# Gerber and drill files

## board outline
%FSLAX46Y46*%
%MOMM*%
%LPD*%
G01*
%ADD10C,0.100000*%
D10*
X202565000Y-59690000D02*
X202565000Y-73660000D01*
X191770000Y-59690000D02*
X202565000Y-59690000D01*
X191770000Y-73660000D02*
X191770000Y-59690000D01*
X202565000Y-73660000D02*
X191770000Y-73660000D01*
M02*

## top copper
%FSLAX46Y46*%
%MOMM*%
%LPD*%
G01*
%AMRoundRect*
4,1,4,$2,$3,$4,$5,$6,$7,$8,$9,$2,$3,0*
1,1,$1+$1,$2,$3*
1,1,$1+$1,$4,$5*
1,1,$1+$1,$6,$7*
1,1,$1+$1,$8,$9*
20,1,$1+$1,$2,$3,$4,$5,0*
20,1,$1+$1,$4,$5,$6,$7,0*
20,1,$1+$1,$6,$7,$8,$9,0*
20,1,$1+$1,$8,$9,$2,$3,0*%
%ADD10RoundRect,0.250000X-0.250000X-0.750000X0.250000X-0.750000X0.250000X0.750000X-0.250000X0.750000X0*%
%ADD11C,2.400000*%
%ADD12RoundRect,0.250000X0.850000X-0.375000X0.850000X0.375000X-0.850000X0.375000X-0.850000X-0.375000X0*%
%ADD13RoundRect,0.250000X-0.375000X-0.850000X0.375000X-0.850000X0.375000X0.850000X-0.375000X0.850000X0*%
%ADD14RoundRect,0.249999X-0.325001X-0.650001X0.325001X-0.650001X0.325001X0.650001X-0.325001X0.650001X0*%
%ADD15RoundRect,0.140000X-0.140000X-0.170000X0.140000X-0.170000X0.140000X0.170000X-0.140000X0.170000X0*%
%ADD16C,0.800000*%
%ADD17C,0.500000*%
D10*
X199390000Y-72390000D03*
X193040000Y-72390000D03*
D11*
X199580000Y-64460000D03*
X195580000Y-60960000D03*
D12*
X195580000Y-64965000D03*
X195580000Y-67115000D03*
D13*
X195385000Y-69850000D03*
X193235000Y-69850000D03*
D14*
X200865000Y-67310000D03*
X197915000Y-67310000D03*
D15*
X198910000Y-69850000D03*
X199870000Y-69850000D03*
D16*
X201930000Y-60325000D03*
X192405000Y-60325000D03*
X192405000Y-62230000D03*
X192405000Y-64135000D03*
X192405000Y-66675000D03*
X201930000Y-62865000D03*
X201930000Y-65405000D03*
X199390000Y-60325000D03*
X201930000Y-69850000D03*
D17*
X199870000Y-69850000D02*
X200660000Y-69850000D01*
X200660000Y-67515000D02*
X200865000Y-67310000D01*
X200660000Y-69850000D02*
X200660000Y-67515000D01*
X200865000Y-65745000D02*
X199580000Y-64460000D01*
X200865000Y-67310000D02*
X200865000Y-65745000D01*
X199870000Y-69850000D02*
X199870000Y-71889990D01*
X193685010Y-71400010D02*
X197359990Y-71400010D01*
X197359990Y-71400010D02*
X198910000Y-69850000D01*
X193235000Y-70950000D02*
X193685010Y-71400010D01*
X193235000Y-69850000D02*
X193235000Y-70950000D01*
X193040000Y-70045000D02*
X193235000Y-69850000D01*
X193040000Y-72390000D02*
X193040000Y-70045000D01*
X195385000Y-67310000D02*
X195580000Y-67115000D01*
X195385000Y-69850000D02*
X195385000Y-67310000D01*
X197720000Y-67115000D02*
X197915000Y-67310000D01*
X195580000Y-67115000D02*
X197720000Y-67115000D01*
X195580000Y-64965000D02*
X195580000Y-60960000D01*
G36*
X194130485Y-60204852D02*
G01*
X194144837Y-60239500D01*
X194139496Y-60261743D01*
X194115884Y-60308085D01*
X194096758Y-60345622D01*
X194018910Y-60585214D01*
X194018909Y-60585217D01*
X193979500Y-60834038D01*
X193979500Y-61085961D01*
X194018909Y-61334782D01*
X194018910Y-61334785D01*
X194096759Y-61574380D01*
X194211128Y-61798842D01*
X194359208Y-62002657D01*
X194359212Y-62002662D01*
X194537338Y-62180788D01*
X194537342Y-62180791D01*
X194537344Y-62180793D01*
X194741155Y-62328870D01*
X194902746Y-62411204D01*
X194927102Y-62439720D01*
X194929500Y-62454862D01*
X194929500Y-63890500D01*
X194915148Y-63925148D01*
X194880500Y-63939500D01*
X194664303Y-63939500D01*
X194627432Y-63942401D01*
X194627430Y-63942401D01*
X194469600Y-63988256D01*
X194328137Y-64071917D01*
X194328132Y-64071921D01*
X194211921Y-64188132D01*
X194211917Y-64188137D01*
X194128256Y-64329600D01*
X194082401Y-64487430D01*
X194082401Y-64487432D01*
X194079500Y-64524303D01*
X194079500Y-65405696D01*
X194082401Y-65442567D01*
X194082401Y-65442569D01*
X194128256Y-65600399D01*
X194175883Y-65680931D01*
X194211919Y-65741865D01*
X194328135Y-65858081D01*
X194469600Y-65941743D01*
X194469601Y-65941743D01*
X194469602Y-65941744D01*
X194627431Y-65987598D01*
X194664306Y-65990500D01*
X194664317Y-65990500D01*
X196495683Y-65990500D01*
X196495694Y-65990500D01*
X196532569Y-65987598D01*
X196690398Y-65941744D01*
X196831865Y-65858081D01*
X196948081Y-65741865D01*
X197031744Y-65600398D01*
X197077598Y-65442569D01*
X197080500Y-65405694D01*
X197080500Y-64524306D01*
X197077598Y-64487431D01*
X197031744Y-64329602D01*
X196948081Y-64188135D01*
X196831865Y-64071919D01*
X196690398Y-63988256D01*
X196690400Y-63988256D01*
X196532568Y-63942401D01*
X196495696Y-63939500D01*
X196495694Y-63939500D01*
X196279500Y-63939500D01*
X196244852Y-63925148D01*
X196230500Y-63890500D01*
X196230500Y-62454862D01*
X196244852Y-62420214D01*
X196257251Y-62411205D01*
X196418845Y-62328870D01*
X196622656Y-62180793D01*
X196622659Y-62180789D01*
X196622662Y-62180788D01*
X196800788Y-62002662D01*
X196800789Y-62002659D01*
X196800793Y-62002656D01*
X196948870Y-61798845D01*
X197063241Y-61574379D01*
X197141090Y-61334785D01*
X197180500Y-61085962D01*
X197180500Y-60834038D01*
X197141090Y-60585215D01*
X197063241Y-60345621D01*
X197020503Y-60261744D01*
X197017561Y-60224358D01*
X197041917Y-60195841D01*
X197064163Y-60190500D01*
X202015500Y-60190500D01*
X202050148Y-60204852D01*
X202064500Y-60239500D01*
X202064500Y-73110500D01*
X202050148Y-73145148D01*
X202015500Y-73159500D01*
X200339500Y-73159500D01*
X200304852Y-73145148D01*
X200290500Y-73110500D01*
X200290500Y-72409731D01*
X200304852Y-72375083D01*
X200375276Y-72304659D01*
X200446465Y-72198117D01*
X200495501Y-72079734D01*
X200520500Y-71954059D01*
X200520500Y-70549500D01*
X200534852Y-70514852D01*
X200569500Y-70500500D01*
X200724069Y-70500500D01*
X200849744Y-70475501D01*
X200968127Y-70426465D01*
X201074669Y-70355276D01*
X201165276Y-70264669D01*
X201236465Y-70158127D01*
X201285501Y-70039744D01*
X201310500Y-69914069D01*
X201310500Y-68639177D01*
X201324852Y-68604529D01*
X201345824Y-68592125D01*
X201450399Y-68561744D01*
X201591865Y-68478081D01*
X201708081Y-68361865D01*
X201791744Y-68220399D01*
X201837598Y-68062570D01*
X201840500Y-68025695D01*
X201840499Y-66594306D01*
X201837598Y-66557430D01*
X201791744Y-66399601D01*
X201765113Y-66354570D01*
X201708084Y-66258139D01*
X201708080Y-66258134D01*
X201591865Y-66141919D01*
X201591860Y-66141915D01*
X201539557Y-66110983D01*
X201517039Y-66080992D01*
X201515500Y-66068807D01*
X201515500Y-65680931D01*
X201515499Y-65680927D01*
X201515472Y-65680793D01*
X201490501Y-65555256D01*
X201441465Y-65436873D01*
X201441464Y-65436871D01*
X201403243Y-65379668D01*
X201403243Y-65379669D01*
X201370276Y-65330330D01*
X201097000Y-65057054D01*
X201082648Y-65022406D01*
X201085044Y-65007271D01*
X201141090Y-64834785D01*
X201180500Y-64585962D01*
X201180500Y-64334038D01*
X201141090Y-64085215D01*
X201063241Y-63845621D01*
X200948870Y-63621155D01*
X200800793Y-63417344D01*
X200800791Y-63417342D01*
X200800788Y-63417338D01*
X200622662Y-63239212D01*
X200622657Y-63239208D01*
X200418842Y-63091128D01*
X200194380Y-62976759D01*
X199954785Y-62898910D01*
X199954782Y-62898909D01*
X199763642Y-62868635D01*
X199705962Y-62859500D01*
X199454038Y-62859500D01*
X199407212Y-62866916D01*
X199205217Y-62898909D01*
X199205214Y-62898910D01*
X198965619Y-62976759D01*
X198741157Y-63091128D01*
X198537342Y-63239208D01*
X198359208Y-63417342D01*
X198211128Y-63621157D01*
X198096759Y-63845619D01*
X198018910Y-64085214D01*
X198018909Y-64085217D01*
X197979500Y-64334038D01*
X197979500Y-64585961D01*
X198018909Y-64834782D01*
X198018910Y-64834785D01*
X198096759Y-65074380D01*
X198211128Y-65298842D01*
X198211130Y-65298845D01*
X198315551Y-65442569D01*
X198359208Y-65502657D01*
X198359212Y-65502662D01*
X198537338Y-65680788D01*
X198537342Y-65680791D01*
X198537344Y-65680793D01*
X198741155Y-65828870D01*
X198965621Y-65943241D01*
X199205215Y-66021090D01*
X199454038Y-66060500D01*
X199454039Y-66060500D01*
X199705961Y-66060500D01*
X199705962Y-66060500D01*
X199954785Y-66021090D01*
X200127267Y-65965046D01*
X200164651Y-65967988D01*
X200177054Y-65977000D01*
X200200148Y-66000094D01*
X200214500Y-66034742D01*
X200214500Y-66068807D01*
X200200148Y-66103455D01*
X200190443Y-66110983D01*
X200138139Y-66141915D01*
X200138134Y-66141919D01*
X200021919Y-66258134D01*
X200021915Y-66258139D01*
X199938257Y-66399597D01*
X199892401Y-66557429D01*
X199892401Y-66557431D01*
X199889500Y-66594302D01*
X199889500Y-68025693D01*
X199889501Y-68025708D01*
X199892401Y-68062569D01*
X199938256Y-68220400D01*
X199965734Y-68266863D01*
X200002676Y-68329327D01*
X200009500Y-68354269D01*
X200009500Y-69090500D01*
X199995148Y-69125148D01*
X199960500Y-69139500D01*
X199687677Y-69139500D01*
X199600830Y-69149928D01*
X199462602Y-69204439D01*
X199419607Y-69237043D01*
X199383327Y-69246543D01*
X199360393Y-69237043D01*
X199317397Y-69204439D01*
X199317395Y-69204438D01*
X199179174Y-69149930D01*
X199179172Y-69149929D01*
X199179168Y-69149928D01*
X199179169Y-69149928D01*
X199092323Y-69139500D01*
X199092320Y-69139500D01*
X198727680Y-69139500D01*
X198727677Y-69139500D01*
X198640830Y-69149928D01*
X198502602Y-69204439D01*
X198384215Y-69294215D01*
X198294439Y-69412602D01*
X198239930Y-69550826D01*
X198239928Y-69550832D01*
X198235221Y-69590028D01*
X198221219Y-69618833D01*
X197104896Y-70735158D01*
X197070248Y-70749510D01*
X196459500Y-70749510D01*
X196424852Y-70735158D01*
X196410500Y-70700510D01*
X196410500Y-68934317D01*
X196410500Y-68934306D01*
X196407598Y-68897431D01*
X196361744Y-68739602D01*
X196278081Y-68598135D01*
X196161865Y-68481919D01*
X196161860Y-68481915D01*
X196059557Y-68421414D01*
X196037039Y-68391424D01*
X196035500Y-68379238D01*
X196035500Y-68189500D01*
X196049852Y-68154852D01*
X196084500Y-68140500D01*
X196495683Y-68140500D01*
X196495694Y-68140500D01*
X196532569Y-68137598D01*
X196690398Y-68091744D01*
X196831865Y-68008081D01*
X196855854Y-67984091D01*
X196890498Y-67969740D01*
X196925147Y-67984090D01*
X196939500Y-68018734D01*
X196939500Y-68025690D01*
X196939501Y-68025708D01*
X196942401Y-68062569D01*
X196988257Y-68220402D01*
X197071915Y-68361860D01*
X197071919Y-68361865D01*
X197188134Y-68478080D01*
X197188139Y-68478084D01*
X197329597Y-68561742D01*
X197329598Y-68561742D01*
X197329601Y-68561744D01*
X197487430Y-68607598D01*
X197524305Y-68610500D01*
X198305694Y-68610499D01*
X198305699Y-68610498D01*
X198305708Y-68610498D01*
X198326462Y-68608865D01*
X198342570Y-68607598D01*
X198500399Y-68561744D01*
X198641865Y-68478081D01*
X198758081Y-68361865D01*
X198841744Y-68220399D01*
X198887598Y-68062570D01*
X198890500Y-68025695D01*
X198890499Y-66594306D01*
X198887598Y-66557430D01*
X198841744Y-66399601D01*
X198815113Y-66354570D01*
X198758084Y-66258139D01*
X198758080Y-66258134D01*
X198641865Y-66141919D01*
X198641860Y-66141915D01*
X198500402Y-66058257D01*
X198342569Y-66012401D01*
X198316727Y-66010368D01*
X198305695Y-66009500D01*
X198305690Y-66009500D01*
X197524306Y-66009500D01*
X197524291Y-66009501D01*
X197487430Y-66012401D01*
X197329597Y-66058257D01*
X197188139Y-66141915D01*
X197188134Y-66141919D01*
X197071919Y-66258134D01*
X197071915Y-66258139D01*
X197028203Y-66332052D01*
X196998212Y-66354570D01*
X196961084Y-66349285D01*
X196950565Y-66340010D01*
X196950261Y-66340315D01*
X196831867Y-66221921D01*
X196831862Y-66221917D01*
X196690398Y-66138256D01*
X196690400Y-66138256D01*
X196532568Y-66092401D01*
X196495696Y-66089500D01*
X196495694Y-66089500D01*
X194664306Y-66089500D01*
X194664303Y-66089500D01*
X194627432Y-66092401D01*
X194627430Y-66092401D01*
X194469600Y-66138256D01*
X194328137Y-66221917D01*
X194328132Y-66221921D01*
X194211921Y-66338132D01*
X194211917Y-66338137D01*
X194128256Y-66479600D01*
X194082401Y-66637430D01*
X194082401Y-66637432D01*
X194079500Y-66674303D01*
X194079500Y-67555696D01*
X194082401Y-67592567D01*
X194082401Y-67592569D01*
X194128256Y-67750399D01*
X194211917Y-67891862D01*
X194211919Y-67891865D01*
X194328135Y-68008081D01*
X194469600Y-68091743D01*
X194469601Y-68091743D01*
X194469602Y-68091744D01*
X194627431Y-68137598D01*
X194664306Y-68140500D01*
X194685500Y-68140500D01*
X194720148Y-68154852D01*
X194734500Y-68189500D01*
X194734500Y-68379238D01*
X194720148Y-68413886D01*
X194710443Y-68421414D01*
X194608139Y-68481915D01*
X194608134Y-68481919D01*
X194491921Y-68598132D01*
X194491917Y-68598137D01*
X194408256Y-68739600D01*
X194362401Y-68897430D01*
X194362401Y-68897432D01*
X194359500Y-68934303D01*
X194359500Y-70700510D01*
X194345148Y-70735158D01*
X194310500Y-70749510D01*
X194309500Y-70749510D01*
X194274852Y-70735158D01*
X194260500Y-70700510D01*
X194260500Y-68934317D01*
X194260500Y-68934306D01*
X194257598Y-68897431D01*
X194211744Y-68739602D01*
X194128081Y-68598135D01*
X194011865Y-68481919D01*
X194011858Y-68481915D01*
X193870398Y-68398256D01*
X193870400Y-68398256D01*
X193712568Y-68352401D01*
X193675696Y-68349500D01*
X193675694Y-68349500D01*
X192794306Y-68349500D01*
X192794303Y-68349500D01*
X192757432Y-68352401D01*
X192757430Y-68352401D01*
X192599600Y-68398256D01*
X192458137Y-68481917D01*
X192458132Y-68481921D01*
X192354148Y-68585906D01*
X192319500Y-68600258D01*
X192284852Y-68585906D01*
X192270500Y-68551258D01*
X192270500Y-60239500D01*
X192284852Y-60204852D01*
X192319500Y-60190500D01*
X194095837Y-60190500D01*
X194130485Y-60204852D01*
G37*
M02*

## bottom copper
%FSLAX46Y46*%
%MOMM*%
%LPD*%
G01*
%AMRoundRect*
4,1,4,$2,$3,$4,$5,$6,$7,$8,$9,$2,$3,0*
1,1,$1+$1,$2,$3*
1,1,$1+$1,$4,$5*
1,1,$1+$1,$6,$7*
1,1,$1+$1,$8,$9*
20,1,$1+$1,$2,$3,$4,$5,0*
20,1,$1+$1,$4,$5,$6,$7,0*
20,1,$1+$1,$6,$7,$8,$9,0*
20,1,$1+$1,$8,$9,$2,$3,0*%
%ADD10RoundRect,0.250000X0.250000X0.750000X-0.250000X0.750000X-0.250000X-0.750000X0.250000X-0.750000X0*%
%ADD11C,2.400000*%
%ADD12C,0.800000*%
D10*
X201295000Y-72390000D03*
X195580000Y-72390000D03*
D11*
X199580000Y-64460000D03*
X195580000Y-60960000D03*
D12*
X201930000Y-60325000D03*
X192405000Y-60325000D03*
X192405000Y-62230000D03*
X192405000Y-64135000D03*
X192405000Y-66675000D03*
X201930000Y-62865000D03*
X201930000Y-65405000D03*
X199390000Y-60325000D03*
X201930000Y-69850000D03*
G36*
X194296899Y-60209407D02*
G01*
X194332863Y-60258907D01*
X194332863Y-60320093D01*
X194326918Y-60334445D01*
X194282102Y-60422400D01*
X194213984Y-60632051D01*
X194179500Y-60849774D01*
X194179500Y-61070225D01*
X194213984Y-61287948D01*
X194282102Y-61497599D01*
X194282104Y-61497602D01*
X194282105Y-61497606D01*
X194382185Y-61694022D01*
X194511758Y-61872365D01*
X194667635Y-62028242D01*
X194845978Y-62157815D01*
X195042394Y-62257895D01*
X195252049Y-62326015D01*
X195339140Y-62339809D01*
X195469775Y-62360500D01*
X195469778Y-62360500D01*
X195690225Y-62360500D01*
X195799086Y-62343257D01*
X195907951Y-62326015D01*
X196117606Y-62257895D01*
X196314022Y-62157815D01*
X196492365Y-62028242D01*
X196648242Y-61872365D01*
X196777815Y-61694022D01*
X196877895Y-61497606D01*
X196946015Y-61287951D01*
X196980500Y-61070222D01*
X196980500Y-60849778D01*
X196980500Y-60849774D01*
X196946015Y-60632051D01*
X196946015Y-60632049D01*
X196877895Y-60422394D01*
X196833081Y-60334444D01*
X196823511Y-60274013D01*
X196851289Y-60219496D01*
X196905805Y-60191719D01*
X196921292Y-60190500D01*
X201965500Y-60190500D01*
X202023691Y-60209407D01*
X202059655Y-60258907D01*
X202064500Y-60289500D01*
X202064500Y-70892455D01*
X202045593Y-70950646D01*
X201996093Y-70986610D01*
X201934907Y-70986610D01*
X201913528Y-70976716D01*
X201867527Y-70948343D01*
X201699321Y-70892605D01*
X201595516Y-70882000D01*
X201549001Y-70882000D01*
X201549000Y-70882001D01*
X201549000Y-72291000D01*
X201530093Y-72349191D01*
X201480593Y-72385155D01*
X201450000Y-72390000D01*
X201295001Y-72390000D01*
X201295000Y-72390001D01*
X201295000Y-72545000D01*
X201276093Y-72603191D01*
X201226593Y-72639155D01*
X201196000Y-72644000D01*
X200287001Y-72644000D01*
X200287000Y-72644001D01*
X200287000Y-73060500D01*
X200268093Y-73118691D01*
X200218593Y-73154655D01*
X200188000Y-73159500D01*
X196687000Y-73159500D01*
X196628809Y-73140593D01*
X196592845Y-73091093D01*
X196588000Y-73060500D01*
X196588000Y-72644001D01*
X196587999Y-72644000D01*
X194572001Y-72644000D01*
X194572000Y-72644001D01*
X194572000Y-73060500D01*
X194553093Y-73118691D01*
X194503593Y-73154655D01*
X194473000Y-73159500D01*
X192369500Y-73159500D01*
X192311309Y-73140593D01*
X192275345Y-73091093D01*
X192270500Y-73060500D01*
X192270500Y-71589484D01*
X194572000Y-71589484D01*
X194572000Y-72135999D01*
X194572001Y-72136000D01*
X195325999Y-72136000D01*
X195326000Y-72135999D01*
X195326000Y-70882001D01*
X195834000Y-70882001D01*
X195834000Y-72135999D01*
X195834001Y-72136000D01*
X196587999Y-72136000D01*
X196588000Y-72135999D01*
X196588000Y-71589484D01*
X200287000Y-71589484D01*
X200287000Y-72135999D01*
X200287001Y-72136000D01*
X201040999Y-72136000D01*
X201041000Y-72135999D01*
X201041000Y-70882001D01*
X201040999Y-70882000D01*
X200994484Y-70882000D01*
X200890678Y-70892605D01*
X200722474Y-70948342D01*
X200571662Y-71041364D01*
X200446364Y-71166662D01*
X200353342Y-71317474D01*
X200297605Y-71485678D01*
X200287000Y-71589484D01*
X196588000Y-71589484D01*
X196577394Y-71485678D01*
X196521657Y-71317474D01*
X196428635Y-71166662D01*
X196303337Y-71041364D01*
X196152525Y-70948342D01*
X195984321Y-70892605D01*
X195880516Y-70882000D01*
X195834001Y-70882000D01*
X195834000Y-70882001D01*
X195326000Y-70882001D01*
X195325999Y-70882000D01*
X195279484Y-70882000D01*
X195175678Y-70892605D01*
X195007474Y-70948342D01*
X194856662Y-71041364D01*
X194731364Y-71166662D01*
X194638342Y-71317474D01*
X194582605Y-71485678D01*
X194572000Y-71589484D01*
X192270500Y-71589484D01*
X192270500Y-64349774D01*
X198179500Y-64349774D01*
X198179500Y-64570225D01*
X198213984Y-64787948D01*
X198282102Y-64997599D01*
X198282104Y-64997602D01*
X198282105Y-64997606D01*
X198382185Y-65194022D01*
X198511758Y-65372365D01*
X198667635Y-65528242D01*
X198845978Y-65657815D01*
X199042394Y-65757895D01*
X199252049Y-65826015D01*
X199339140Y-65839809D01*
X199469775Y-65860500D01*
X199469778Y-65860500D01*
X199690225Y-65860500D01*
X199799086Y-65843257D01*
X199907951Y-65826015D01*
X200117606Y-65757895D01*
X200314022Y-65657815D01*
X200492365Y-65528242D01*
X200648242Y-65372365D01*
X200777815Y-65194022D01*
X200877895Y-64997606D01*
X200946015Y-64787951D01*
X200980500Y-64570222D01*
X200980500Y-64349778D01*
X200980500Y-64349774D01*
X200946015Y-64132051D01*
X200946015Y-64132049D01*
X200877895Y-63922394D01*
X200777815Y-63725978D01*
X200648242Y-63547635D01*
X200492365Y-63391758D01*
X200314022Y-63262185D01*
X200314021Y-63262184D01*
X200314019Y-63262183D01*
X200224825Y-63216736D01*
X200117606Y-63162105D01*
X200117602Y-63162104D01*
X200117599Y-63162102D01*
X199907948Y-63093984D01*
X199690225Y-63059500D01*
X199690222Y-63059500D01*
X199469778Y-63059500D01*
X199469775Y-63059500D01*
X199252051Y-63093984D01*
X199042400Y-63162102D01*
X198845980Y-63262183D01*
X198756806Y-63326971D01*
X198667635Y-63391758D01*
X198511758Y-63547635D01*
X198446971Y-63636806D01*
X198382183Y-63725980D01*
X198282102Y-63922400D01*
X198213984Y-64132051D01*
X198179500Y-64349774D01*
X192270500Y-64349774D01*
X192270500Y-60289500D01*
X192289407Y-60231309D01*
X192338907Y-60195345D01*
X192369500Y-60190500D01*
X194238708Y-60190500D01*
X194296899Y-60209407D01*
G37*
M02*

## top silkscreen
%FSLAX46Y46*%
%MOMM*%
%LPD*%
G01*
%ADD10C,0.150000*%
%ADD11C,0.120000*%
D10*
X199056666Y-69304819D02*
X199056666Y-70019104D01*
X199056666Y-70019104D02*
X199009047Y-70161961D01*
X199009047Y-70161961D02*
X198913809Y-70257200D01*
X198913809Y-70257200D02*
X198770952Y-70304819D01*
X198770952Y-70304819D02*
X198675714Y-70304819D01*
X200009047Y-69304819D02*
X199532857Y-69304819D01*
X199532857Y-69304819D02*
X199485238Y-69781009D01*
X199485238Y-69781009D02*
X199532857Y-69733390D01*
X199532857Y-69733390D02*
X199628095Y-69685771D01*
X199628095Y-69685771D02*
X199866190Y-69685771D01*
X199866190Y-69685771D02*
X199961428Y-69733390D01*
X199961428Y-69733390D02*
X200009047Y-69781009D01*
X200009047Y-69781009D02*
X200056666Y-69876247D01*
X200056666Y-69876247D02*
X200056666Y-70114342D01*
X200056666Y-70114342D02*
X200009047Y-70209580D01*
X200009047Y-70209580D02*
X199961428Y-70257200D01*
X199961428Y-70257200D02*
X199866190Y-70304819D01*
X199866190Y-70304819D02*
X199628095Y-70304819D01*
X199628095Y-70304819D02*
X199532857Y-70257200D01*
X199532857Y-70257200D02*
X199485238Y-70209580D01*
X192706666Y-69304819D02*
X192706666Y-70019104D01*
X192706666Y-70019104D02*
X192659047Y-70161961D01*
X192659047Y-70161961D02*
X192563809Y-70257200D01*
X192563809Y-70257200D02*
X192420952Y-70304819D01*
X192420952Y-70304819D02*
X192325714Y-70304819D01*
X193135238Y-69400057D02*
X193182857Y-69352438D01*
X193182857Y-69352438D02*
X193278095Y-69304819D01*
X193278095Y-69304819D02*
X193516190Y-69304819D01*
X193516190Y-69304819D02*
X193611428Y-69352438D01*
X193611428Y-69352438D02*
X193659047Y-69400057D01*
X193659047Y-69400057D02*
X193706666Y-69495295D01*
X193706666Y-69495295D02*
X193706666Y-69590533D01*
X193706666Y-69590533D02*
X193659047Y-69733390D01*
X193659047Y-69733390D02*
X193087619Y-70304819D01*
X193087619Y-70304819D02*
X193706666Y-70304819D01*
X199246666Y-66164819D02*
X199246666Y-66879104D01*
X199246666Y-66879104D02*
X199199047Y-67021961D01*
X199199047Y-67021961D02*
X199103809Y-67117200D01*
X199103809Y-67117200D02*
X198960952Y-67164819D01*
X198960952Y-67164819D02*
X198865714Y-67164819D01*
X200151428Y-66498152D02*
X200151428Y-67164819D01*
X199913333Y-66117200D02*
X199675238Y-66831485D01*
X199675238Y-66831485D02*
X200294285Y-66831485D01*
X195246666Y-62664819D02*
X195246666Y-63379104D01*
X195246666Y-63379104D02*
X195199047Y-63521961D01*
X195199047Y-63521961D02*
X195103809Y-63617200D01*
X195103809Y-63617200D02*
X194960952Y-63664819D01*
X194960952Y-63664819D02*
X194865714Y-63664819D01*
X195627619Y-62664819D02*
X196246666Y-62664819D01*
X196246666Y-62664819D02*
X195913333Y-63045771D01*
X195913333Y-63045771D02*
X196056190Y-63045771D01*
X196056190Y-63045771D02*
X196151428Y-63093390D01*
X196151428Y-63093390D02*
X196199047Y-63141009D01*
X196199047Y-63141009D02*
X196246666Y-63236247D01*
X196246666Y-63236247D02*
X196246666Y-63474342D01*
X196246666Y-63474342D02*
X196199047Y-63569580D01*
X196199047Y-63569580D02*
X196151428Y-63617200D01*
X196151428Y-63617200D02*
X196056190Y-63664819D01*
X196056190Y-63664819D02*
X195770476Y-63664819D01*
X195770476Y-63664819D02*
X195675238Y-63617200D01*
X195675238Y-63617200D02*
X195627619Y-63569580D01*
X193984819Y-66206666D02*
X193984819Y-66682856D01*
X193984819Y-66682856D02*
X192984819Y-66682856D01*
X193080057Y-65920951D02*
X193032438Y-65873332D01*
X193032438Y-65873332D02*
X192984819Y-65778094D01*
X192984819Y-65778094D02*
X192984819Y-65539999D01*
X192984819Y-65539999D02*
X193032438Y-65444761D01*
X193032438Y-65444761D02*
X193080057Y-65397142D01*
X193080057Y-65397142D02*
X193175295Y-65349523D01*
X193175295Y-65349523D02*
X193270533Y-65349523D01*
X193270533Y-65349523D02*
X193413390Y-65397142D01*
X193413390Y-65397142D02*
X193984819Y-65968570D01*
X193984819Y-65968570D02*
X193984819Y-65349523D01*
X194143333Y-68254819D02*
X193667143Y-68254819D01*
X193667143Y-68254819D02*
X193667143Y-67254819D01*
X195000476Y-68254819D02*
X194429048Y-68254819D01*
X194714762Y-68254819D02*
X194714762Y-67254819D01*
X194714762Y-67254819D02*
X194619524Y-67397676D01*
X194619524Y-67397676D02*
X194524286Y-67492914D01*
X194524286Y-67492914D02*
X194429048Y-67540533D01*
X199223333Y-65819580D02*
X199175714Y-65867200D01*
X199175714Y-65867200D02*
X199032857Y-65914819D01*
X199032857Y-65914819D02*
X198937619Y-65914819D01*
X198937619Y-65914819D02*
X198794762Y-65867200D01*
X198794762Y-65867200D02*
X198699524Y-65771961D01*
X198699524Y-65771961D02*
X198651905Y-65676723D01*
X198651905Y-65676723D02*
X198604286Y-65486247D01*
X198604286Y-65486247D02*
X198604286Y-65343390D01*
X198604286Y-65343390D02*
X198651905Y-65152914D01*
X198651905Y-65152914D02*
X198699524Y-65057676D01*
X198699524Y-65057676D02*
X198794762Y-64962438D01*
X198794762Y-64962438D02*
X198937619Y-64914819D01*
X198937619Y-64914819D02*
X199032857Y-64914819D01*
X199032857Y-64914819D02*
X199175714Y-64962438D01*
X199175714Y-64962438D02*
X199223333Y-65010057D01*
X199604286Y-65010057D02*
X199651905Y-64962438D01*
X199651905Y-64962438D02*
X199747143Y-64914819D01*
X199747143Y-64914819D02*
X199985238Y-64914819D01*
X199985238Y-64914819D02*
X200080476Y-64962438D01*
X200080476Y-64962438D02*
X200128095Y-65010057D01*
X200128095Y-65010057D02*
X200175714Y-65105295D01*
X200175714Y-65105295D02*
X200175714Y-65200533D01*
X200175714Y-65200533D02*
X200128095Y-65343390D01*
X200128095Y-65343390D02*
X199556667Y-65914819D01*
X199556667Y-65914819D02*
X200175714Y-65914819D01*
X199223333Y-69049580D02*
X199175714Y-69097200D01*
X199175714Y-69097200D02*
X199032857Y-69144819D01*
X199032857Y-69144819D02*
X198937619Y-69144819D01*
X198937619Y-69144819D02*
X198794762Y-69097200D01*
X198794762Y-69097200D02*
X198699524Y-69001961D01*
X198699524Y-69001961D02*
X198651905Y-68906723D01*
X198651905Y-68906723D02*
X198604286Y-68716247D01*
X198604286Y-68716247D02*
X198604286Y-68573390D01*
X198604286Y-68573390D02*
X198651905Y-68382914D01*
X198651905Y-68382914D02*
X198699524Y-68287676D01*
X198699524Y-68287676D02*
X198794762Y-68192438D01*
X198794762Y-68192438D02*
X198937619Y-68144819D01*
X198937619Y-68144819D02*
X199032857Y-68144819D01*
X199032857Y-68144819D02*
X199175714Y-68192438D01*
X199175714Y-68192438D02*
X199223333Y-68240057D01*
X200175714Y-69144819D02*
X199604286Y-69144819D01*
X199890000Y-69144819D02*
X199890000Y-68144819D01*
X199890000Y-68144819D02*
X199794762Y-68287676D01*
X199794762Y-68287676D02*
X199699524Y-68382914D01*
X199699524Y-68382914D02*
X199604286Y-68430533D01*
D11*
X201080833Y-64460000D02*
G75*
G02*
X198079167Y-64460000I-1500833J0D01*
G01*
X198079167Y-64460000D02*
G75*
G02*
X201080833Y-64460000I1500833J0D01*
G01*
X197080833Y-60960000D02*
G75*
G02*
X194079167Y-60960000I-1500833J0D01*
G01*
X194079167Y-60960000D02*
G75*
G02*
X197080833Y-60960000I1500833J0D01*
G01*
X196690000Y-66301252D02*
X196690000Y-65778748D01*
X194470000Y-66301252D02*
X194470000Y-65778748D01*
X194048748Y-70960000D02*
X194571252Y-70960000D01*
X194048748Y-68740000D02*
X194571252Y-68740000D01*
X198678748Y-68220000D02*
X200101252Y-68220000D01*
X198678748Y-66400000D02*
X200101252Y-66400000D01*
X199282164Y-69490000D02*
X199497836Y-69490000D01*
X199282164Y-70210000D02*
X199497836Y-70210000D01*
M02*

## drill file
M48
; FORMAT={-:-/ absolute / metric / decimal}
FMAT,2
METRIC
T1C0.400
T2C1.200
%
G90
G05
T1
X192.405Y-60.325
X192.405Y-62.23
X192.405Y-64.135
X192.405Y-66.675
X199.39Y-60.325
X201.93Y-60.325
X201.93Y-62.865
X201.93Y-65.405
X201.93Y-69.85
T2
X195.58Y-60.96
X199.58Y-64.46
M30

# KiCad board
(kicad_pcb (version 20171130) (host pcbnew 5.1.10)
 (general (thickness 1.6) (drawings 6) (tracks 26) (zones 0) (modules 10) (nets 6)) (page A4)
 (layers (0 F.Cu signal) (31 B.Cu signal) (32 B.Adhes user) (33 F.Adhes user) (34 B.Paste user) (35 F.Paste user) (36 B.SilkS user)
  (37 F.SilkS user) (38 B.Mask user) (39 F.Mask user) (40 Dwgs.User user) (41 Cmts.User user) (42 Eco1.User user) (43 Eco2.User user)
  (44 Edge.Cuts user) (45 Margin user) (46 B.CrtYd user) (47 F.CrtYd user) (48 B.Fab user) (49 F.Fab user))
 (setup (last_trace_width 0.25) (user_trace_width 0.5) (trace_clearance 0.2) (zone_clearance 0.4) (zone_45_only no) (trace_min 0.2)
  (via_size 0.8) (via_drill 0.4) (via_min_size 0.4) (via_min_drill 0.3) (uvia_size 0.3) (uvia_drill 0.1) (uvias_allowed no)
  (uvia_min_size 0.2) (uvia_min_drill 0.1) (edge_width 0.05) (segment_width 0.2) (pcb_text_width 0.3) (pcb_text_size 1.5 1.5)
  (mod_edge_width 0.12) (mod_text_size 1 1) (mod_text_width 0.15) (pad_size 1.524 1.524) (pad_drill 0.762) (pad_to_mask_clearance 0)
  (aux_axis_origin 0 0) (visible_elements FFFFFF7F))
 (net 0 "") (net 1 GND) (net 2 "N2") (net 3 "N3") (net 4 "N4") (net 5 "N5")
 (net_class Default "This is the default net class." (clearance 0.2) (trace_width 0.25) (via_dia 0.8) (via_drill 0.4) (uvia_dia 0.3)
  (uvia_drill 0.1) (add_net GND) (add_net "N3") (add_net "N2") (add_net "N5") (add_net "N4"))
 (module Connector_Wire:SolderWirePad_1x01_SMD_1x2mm (layer B.Cu) (at 201.295 72.39 180)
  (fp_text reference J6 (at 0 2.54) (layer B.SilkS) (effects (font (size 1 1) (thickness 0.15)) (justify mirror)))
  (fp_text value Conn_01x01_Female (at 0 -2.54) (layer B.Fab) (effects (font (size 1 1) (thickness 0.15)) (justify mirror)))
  (pad 1 smd roundrect (at 0 0 180) (size 1 2) (layers B.Cu B.Paste B.Mask) (roundrect_rratio 0.25) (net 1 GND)))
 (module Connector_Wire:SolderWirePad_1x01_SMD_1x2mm (layer F.Cu) (at 199.39 72.39)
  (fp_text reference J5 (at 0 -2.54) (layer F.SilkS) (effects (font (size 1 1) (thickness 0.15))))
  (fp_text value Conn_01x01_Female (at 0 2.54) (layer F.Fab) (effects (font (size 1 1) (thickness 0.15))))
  (pad 1 smd roundrect (at 0 0) (size 1 2) (layers F.Cu F.Paste F.Mask) (roundrect_rratio 0.25) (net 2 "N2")))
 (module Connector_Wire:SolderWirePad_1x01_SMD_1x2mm (layer F.Cu) (at 193.04 72.39)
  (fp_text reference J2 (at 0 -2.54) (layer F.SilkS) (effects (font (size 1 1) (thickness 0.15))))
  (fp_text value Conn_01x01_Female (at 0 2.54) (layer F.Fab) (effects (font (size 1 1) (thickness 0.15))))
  (pad 1 smd roundrect (at 0 0) (size 1 2) (layers F.Cu F.Paste F.Mask) (roundrect_rratio 0.25) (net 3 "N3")))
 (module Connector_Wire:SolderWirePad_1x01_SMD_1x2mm (layer B.Cu) (at 195.58 72.39 180)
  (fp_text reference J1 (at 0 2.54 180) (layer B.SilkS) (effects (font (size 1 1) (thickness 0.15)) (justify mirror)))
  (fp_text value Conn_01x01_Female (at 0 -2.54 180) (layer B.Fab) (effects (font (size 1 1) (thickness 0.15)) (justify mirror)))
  (pad 1 smd roundrect (at 0 0 180) (size 1 2) (layers B.Cu B.Paste B.Mask) (roundrect_rratio 0.25) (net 1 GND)))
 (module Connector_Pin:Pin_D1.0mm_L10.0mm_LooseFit (layer F.Cu) (at 199.58 64.46)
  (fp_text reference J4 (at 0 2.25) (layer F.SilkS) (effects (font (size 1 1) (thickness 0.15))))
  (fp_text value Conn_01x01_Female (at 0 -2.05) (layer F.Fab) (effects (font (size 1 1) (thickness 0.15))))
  (fp_circle (center 0 0) (end 1.5 0.05) (layer F.SilkS) (width 0.12))
  (pad 1 thru_hole circle (at 0 0) (size 2.4 2.4) (drill 1.2) (layers *.Cu *.Mask) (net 2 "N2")))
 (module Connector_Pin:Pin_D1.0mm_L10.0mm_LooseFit (layer F.Cu) (at 195.58 60.96)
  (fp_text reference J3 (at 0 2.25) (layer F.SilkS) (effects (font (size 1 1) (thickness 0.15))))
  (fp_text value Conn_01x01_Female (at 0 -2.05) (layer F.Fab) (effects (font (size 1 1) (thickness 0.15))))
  (fp_circle (center 0 0) (end 1.5 0.05) (layer F.SilkS) (width 0.12))
  (pad 1 thru_hole circle (at 0 0) (size 2.4 2.4) (drill 1.2) (layers *.Cu *.Mask) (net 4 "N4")))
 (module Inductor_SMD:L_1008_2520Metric (layer F.Cu) (at 195.58 66.04 90)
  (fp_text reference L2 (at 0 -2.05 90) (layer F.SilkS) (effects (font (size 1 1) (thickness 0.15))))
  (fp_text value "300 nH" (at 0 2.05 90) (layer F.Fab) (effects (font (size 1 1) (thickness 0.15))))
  (fp_line (start -0.261252 1.11) (end 0.261252 1.11) (layer F.SilkS) (width 0.12))
  (fp_line (start -0.261252 -1.11) (end 0.261252 -1.11) (layer F.SilkS) (width 0.12))
  (pad 2 smd roundrect (at 1.075 0 90) (size 1.25 2.2) (layers F.Cu F.Paste F.Mask) (roundrect_rratio 0.2) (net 4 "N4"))
  (pad 1 smd roundrect (at -1.075 0 90) (size 1.25 2.2) (layers F.Cu F.Paste F.Mask) (roundrect_rratio 0.2) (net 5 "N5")))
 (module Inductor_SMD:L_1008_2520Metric (layer F.Cu) (at 194.31 69.85)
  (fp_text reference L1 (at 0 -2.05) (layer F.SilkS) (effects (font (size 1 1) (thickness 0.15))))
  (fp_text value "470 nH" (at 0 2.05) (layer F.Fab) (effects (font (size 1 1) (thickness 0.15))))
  (fp_line (start -0.261252 1.11) (end 0.261252 1.11) (layer F.SilkS) (width 0.12))
  (fp_line (start -0.261252 -1.11) (end 0.261252 -1.11) (layer F.SilkS) (width 0.12))
  (pad 2 smd roundrect (at 1.075 0) (size 1.25 2.2) (layers F.Cu F.Paste F.Mask) (roundrect_rratio 0.2) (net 5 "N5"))
  (pad 1 smd roundrect (at -1.075 0) (size 1.25 2.2) (layers F.Cu F.Paste F.Mask) (roundrect_rratio 0.2) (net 3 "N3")))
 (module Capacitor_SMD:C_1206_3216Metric (layer F.Cu) (at 199.39 67.31)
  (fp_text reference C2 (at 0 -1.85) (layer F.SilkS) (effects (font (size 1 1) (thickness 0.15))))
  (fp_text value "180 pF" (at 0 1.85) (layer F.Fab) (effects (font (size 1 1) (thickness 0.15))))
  (fp_line (start -0.711252 0.91) (end 0.711252 0.91) (layer F.SilkS) (width 0.12))
  (fp_line (start -0.711252 -0.91) (end 0.711252 -0.91) (layer F.SilkS) (width 0.12))
  (pad 2 smd roundrect (at 1.475 0) (size 1.15 1.8) (layers F.Cu F.Paste F.Mask) (roundrect_rratio 0.2173904347826087) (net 2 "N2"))
  (pad 1 smd roundrect (at -1.475 0) (size 1.15 1.8) (layers F.Cu F.Paste F.Mask) (roundrect_rratio 0.2173904347826087) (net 5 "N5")))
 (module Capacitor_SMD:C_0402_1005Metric (layer F.Cu) (at 199.39 69.85)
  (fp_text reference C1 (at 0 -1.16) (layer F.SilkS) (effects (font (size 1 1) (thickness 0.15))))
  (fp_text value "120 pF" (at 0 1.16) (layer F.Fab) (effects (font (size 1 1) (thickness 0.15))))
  (fp_line (start -0.107836 -0.36) (end 0.107836 -0.36) (layer F.SilkS) (width 0.12))
  (fp_line (start -0.107836 0.36) (end 0.107836 0.36) (layer F.SilkS) (width 0.12))
  (pad 1 smd roundrect (at -0.48 0) (size 0.56 0.62) (layers F.Cu F.Paste F.Mask) (roundrect_rratio 0.25) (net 3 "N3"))
  (pad 2 smd roundrect (at 0.48 0) (size 0.56 0.62) (layers F.Cu F.Paste F.Mask) (roundrect_rratio 0.25) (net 2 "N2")))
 (gr_line (start 202.565 59.69) (end 202.565 73.66) (layer Edge.Cuts) (width 0.1))
 (gr_line (start 191.77 59.69) (end 202.565 59.69) (layer Edge.Cuts) (width 0.1))
 (gr_line (start 191.77 73.66) (end 191.77 59.69) (layer Edge.Cuts) (width 0.1))
 (gr_line (start 202.565 73.66) (end 191.77 73.66) (layer Edge.Cuts) (width 0.1))
 (via (at 201.93 60.325) (size 0.8) (drill 0.4) (layers F.Cu B.Cu) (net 1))
 (via (at 192.405 60.325) (size 0.8) (drill 0.4) (layers F.Cu B.Cu) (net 1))
 (via (at 192.405 62.23) (size 0.8) (drill 0.4) (layers F.Cu B.Cu) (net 1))
 (via (at 192.405 64.135) (size 0.8) (drill 0.4) (layers F.Cu B.Cu) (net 1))
 (via (at 192.405 66.675) (size 0.8) (drill 0.4) (layers F.Cu B.Cu) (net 1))
 (via (at 201.93 62.865) (size 0.8) (drill 0.4) (layers F.Cu B.Cu) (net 1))
 (via (at 201.93 65.405) (size 0.8) (drill 0.4) (layers F.Cu B.Cu) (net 1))
 (via (at 199.39 60.325) (size 0.8) (drill 0.4) (layers F.Cu B.Cu) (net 1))
 (via (at 201.93 69.85) (size 0.8) (drill 0.4) (layers F.Cu B.Cu) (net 1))
 (segment (start 199.87 69.85) (end 200.66 69.85) (width 0.5) (layer F.Cu) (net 2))
 (segment (start 200.66 67.515) (end 200.865 67.31) (width 0.5) (layer F.Cu) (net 2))
 (segment (start 200.66 69.85) (end 200.66 67.515) (width 0.5) (layer F.Cu) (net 2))
 (segment (start 200.865 65.745) (end 199.58 64.46) (width 0.5) (layer F.Cu) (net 2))
 (segment (start 200.865 67.31) (end 200.865 65.745) (width 0.5) (layer F.Cu) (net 2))
 (segment (start 199.87 69.85) (end 199.87 71.88999) (width 0.5) (layer F.Cu) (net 2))
 (segment (start 193.68501 71.40001) (end 197.35999 71.40001) (width 0.5) (layer F.Cu) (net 3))
 (segment (start 197.35999 71.40001) (end 198.91 69.85) (width 0.5) (layer F.Cu) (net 3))
 (segment (start 193.235 70.95) (end 193.68501 71.40001) (width 0.5) (layer F.Cu) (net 3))
 (segment (start 193.235 69.85) (end 193.235 70.95) (width 0.5) (layer F.Cu) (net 3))
 (segment (start 193.04 70.045) (end 193.235 69.85) (width 0.5) (layer F.Cu) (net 3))
 (segment (start 193.04 72.39) (end 193.04 70.045) (width 0.5) (layer F.Cu) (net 3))
 (segment (start 195.385 67.31) (end 195.58 67.115) (width 0.5) (layer F.Cu) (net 5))
 (segment (start 195.385 69.85) (end 195.385 67.31) (width 0.5) (layer F.Cu) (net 5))
 (segment (start 197.72 67.115) (end 197.915 67.31) (width 0.5) (layer F.Cu) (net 5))
 (segment (start 195.58 67.115) (end 197.72 67.115) (width 0.5) (layer F.Cu) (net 5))
 (segment (start 195.58 64.965) (end 195.58 60.96) (width 0.5) (layer F.Cu) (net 4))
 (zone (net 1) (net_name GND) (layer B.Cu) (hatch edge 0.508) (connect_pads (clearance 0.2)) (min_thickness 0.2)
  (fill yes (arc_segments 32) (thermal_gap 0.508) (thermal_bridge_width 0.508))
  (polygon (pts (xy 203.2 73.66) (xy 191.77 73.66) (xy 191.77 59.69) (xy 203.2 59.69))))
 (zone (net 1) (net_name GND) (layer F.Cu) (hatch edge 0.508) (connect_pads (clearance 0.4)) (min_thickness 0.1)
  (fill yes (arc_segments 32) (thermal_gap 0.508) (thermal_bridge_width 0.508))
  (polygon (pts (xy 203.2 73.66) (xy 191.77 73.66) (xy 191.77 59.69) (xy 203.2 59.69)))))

